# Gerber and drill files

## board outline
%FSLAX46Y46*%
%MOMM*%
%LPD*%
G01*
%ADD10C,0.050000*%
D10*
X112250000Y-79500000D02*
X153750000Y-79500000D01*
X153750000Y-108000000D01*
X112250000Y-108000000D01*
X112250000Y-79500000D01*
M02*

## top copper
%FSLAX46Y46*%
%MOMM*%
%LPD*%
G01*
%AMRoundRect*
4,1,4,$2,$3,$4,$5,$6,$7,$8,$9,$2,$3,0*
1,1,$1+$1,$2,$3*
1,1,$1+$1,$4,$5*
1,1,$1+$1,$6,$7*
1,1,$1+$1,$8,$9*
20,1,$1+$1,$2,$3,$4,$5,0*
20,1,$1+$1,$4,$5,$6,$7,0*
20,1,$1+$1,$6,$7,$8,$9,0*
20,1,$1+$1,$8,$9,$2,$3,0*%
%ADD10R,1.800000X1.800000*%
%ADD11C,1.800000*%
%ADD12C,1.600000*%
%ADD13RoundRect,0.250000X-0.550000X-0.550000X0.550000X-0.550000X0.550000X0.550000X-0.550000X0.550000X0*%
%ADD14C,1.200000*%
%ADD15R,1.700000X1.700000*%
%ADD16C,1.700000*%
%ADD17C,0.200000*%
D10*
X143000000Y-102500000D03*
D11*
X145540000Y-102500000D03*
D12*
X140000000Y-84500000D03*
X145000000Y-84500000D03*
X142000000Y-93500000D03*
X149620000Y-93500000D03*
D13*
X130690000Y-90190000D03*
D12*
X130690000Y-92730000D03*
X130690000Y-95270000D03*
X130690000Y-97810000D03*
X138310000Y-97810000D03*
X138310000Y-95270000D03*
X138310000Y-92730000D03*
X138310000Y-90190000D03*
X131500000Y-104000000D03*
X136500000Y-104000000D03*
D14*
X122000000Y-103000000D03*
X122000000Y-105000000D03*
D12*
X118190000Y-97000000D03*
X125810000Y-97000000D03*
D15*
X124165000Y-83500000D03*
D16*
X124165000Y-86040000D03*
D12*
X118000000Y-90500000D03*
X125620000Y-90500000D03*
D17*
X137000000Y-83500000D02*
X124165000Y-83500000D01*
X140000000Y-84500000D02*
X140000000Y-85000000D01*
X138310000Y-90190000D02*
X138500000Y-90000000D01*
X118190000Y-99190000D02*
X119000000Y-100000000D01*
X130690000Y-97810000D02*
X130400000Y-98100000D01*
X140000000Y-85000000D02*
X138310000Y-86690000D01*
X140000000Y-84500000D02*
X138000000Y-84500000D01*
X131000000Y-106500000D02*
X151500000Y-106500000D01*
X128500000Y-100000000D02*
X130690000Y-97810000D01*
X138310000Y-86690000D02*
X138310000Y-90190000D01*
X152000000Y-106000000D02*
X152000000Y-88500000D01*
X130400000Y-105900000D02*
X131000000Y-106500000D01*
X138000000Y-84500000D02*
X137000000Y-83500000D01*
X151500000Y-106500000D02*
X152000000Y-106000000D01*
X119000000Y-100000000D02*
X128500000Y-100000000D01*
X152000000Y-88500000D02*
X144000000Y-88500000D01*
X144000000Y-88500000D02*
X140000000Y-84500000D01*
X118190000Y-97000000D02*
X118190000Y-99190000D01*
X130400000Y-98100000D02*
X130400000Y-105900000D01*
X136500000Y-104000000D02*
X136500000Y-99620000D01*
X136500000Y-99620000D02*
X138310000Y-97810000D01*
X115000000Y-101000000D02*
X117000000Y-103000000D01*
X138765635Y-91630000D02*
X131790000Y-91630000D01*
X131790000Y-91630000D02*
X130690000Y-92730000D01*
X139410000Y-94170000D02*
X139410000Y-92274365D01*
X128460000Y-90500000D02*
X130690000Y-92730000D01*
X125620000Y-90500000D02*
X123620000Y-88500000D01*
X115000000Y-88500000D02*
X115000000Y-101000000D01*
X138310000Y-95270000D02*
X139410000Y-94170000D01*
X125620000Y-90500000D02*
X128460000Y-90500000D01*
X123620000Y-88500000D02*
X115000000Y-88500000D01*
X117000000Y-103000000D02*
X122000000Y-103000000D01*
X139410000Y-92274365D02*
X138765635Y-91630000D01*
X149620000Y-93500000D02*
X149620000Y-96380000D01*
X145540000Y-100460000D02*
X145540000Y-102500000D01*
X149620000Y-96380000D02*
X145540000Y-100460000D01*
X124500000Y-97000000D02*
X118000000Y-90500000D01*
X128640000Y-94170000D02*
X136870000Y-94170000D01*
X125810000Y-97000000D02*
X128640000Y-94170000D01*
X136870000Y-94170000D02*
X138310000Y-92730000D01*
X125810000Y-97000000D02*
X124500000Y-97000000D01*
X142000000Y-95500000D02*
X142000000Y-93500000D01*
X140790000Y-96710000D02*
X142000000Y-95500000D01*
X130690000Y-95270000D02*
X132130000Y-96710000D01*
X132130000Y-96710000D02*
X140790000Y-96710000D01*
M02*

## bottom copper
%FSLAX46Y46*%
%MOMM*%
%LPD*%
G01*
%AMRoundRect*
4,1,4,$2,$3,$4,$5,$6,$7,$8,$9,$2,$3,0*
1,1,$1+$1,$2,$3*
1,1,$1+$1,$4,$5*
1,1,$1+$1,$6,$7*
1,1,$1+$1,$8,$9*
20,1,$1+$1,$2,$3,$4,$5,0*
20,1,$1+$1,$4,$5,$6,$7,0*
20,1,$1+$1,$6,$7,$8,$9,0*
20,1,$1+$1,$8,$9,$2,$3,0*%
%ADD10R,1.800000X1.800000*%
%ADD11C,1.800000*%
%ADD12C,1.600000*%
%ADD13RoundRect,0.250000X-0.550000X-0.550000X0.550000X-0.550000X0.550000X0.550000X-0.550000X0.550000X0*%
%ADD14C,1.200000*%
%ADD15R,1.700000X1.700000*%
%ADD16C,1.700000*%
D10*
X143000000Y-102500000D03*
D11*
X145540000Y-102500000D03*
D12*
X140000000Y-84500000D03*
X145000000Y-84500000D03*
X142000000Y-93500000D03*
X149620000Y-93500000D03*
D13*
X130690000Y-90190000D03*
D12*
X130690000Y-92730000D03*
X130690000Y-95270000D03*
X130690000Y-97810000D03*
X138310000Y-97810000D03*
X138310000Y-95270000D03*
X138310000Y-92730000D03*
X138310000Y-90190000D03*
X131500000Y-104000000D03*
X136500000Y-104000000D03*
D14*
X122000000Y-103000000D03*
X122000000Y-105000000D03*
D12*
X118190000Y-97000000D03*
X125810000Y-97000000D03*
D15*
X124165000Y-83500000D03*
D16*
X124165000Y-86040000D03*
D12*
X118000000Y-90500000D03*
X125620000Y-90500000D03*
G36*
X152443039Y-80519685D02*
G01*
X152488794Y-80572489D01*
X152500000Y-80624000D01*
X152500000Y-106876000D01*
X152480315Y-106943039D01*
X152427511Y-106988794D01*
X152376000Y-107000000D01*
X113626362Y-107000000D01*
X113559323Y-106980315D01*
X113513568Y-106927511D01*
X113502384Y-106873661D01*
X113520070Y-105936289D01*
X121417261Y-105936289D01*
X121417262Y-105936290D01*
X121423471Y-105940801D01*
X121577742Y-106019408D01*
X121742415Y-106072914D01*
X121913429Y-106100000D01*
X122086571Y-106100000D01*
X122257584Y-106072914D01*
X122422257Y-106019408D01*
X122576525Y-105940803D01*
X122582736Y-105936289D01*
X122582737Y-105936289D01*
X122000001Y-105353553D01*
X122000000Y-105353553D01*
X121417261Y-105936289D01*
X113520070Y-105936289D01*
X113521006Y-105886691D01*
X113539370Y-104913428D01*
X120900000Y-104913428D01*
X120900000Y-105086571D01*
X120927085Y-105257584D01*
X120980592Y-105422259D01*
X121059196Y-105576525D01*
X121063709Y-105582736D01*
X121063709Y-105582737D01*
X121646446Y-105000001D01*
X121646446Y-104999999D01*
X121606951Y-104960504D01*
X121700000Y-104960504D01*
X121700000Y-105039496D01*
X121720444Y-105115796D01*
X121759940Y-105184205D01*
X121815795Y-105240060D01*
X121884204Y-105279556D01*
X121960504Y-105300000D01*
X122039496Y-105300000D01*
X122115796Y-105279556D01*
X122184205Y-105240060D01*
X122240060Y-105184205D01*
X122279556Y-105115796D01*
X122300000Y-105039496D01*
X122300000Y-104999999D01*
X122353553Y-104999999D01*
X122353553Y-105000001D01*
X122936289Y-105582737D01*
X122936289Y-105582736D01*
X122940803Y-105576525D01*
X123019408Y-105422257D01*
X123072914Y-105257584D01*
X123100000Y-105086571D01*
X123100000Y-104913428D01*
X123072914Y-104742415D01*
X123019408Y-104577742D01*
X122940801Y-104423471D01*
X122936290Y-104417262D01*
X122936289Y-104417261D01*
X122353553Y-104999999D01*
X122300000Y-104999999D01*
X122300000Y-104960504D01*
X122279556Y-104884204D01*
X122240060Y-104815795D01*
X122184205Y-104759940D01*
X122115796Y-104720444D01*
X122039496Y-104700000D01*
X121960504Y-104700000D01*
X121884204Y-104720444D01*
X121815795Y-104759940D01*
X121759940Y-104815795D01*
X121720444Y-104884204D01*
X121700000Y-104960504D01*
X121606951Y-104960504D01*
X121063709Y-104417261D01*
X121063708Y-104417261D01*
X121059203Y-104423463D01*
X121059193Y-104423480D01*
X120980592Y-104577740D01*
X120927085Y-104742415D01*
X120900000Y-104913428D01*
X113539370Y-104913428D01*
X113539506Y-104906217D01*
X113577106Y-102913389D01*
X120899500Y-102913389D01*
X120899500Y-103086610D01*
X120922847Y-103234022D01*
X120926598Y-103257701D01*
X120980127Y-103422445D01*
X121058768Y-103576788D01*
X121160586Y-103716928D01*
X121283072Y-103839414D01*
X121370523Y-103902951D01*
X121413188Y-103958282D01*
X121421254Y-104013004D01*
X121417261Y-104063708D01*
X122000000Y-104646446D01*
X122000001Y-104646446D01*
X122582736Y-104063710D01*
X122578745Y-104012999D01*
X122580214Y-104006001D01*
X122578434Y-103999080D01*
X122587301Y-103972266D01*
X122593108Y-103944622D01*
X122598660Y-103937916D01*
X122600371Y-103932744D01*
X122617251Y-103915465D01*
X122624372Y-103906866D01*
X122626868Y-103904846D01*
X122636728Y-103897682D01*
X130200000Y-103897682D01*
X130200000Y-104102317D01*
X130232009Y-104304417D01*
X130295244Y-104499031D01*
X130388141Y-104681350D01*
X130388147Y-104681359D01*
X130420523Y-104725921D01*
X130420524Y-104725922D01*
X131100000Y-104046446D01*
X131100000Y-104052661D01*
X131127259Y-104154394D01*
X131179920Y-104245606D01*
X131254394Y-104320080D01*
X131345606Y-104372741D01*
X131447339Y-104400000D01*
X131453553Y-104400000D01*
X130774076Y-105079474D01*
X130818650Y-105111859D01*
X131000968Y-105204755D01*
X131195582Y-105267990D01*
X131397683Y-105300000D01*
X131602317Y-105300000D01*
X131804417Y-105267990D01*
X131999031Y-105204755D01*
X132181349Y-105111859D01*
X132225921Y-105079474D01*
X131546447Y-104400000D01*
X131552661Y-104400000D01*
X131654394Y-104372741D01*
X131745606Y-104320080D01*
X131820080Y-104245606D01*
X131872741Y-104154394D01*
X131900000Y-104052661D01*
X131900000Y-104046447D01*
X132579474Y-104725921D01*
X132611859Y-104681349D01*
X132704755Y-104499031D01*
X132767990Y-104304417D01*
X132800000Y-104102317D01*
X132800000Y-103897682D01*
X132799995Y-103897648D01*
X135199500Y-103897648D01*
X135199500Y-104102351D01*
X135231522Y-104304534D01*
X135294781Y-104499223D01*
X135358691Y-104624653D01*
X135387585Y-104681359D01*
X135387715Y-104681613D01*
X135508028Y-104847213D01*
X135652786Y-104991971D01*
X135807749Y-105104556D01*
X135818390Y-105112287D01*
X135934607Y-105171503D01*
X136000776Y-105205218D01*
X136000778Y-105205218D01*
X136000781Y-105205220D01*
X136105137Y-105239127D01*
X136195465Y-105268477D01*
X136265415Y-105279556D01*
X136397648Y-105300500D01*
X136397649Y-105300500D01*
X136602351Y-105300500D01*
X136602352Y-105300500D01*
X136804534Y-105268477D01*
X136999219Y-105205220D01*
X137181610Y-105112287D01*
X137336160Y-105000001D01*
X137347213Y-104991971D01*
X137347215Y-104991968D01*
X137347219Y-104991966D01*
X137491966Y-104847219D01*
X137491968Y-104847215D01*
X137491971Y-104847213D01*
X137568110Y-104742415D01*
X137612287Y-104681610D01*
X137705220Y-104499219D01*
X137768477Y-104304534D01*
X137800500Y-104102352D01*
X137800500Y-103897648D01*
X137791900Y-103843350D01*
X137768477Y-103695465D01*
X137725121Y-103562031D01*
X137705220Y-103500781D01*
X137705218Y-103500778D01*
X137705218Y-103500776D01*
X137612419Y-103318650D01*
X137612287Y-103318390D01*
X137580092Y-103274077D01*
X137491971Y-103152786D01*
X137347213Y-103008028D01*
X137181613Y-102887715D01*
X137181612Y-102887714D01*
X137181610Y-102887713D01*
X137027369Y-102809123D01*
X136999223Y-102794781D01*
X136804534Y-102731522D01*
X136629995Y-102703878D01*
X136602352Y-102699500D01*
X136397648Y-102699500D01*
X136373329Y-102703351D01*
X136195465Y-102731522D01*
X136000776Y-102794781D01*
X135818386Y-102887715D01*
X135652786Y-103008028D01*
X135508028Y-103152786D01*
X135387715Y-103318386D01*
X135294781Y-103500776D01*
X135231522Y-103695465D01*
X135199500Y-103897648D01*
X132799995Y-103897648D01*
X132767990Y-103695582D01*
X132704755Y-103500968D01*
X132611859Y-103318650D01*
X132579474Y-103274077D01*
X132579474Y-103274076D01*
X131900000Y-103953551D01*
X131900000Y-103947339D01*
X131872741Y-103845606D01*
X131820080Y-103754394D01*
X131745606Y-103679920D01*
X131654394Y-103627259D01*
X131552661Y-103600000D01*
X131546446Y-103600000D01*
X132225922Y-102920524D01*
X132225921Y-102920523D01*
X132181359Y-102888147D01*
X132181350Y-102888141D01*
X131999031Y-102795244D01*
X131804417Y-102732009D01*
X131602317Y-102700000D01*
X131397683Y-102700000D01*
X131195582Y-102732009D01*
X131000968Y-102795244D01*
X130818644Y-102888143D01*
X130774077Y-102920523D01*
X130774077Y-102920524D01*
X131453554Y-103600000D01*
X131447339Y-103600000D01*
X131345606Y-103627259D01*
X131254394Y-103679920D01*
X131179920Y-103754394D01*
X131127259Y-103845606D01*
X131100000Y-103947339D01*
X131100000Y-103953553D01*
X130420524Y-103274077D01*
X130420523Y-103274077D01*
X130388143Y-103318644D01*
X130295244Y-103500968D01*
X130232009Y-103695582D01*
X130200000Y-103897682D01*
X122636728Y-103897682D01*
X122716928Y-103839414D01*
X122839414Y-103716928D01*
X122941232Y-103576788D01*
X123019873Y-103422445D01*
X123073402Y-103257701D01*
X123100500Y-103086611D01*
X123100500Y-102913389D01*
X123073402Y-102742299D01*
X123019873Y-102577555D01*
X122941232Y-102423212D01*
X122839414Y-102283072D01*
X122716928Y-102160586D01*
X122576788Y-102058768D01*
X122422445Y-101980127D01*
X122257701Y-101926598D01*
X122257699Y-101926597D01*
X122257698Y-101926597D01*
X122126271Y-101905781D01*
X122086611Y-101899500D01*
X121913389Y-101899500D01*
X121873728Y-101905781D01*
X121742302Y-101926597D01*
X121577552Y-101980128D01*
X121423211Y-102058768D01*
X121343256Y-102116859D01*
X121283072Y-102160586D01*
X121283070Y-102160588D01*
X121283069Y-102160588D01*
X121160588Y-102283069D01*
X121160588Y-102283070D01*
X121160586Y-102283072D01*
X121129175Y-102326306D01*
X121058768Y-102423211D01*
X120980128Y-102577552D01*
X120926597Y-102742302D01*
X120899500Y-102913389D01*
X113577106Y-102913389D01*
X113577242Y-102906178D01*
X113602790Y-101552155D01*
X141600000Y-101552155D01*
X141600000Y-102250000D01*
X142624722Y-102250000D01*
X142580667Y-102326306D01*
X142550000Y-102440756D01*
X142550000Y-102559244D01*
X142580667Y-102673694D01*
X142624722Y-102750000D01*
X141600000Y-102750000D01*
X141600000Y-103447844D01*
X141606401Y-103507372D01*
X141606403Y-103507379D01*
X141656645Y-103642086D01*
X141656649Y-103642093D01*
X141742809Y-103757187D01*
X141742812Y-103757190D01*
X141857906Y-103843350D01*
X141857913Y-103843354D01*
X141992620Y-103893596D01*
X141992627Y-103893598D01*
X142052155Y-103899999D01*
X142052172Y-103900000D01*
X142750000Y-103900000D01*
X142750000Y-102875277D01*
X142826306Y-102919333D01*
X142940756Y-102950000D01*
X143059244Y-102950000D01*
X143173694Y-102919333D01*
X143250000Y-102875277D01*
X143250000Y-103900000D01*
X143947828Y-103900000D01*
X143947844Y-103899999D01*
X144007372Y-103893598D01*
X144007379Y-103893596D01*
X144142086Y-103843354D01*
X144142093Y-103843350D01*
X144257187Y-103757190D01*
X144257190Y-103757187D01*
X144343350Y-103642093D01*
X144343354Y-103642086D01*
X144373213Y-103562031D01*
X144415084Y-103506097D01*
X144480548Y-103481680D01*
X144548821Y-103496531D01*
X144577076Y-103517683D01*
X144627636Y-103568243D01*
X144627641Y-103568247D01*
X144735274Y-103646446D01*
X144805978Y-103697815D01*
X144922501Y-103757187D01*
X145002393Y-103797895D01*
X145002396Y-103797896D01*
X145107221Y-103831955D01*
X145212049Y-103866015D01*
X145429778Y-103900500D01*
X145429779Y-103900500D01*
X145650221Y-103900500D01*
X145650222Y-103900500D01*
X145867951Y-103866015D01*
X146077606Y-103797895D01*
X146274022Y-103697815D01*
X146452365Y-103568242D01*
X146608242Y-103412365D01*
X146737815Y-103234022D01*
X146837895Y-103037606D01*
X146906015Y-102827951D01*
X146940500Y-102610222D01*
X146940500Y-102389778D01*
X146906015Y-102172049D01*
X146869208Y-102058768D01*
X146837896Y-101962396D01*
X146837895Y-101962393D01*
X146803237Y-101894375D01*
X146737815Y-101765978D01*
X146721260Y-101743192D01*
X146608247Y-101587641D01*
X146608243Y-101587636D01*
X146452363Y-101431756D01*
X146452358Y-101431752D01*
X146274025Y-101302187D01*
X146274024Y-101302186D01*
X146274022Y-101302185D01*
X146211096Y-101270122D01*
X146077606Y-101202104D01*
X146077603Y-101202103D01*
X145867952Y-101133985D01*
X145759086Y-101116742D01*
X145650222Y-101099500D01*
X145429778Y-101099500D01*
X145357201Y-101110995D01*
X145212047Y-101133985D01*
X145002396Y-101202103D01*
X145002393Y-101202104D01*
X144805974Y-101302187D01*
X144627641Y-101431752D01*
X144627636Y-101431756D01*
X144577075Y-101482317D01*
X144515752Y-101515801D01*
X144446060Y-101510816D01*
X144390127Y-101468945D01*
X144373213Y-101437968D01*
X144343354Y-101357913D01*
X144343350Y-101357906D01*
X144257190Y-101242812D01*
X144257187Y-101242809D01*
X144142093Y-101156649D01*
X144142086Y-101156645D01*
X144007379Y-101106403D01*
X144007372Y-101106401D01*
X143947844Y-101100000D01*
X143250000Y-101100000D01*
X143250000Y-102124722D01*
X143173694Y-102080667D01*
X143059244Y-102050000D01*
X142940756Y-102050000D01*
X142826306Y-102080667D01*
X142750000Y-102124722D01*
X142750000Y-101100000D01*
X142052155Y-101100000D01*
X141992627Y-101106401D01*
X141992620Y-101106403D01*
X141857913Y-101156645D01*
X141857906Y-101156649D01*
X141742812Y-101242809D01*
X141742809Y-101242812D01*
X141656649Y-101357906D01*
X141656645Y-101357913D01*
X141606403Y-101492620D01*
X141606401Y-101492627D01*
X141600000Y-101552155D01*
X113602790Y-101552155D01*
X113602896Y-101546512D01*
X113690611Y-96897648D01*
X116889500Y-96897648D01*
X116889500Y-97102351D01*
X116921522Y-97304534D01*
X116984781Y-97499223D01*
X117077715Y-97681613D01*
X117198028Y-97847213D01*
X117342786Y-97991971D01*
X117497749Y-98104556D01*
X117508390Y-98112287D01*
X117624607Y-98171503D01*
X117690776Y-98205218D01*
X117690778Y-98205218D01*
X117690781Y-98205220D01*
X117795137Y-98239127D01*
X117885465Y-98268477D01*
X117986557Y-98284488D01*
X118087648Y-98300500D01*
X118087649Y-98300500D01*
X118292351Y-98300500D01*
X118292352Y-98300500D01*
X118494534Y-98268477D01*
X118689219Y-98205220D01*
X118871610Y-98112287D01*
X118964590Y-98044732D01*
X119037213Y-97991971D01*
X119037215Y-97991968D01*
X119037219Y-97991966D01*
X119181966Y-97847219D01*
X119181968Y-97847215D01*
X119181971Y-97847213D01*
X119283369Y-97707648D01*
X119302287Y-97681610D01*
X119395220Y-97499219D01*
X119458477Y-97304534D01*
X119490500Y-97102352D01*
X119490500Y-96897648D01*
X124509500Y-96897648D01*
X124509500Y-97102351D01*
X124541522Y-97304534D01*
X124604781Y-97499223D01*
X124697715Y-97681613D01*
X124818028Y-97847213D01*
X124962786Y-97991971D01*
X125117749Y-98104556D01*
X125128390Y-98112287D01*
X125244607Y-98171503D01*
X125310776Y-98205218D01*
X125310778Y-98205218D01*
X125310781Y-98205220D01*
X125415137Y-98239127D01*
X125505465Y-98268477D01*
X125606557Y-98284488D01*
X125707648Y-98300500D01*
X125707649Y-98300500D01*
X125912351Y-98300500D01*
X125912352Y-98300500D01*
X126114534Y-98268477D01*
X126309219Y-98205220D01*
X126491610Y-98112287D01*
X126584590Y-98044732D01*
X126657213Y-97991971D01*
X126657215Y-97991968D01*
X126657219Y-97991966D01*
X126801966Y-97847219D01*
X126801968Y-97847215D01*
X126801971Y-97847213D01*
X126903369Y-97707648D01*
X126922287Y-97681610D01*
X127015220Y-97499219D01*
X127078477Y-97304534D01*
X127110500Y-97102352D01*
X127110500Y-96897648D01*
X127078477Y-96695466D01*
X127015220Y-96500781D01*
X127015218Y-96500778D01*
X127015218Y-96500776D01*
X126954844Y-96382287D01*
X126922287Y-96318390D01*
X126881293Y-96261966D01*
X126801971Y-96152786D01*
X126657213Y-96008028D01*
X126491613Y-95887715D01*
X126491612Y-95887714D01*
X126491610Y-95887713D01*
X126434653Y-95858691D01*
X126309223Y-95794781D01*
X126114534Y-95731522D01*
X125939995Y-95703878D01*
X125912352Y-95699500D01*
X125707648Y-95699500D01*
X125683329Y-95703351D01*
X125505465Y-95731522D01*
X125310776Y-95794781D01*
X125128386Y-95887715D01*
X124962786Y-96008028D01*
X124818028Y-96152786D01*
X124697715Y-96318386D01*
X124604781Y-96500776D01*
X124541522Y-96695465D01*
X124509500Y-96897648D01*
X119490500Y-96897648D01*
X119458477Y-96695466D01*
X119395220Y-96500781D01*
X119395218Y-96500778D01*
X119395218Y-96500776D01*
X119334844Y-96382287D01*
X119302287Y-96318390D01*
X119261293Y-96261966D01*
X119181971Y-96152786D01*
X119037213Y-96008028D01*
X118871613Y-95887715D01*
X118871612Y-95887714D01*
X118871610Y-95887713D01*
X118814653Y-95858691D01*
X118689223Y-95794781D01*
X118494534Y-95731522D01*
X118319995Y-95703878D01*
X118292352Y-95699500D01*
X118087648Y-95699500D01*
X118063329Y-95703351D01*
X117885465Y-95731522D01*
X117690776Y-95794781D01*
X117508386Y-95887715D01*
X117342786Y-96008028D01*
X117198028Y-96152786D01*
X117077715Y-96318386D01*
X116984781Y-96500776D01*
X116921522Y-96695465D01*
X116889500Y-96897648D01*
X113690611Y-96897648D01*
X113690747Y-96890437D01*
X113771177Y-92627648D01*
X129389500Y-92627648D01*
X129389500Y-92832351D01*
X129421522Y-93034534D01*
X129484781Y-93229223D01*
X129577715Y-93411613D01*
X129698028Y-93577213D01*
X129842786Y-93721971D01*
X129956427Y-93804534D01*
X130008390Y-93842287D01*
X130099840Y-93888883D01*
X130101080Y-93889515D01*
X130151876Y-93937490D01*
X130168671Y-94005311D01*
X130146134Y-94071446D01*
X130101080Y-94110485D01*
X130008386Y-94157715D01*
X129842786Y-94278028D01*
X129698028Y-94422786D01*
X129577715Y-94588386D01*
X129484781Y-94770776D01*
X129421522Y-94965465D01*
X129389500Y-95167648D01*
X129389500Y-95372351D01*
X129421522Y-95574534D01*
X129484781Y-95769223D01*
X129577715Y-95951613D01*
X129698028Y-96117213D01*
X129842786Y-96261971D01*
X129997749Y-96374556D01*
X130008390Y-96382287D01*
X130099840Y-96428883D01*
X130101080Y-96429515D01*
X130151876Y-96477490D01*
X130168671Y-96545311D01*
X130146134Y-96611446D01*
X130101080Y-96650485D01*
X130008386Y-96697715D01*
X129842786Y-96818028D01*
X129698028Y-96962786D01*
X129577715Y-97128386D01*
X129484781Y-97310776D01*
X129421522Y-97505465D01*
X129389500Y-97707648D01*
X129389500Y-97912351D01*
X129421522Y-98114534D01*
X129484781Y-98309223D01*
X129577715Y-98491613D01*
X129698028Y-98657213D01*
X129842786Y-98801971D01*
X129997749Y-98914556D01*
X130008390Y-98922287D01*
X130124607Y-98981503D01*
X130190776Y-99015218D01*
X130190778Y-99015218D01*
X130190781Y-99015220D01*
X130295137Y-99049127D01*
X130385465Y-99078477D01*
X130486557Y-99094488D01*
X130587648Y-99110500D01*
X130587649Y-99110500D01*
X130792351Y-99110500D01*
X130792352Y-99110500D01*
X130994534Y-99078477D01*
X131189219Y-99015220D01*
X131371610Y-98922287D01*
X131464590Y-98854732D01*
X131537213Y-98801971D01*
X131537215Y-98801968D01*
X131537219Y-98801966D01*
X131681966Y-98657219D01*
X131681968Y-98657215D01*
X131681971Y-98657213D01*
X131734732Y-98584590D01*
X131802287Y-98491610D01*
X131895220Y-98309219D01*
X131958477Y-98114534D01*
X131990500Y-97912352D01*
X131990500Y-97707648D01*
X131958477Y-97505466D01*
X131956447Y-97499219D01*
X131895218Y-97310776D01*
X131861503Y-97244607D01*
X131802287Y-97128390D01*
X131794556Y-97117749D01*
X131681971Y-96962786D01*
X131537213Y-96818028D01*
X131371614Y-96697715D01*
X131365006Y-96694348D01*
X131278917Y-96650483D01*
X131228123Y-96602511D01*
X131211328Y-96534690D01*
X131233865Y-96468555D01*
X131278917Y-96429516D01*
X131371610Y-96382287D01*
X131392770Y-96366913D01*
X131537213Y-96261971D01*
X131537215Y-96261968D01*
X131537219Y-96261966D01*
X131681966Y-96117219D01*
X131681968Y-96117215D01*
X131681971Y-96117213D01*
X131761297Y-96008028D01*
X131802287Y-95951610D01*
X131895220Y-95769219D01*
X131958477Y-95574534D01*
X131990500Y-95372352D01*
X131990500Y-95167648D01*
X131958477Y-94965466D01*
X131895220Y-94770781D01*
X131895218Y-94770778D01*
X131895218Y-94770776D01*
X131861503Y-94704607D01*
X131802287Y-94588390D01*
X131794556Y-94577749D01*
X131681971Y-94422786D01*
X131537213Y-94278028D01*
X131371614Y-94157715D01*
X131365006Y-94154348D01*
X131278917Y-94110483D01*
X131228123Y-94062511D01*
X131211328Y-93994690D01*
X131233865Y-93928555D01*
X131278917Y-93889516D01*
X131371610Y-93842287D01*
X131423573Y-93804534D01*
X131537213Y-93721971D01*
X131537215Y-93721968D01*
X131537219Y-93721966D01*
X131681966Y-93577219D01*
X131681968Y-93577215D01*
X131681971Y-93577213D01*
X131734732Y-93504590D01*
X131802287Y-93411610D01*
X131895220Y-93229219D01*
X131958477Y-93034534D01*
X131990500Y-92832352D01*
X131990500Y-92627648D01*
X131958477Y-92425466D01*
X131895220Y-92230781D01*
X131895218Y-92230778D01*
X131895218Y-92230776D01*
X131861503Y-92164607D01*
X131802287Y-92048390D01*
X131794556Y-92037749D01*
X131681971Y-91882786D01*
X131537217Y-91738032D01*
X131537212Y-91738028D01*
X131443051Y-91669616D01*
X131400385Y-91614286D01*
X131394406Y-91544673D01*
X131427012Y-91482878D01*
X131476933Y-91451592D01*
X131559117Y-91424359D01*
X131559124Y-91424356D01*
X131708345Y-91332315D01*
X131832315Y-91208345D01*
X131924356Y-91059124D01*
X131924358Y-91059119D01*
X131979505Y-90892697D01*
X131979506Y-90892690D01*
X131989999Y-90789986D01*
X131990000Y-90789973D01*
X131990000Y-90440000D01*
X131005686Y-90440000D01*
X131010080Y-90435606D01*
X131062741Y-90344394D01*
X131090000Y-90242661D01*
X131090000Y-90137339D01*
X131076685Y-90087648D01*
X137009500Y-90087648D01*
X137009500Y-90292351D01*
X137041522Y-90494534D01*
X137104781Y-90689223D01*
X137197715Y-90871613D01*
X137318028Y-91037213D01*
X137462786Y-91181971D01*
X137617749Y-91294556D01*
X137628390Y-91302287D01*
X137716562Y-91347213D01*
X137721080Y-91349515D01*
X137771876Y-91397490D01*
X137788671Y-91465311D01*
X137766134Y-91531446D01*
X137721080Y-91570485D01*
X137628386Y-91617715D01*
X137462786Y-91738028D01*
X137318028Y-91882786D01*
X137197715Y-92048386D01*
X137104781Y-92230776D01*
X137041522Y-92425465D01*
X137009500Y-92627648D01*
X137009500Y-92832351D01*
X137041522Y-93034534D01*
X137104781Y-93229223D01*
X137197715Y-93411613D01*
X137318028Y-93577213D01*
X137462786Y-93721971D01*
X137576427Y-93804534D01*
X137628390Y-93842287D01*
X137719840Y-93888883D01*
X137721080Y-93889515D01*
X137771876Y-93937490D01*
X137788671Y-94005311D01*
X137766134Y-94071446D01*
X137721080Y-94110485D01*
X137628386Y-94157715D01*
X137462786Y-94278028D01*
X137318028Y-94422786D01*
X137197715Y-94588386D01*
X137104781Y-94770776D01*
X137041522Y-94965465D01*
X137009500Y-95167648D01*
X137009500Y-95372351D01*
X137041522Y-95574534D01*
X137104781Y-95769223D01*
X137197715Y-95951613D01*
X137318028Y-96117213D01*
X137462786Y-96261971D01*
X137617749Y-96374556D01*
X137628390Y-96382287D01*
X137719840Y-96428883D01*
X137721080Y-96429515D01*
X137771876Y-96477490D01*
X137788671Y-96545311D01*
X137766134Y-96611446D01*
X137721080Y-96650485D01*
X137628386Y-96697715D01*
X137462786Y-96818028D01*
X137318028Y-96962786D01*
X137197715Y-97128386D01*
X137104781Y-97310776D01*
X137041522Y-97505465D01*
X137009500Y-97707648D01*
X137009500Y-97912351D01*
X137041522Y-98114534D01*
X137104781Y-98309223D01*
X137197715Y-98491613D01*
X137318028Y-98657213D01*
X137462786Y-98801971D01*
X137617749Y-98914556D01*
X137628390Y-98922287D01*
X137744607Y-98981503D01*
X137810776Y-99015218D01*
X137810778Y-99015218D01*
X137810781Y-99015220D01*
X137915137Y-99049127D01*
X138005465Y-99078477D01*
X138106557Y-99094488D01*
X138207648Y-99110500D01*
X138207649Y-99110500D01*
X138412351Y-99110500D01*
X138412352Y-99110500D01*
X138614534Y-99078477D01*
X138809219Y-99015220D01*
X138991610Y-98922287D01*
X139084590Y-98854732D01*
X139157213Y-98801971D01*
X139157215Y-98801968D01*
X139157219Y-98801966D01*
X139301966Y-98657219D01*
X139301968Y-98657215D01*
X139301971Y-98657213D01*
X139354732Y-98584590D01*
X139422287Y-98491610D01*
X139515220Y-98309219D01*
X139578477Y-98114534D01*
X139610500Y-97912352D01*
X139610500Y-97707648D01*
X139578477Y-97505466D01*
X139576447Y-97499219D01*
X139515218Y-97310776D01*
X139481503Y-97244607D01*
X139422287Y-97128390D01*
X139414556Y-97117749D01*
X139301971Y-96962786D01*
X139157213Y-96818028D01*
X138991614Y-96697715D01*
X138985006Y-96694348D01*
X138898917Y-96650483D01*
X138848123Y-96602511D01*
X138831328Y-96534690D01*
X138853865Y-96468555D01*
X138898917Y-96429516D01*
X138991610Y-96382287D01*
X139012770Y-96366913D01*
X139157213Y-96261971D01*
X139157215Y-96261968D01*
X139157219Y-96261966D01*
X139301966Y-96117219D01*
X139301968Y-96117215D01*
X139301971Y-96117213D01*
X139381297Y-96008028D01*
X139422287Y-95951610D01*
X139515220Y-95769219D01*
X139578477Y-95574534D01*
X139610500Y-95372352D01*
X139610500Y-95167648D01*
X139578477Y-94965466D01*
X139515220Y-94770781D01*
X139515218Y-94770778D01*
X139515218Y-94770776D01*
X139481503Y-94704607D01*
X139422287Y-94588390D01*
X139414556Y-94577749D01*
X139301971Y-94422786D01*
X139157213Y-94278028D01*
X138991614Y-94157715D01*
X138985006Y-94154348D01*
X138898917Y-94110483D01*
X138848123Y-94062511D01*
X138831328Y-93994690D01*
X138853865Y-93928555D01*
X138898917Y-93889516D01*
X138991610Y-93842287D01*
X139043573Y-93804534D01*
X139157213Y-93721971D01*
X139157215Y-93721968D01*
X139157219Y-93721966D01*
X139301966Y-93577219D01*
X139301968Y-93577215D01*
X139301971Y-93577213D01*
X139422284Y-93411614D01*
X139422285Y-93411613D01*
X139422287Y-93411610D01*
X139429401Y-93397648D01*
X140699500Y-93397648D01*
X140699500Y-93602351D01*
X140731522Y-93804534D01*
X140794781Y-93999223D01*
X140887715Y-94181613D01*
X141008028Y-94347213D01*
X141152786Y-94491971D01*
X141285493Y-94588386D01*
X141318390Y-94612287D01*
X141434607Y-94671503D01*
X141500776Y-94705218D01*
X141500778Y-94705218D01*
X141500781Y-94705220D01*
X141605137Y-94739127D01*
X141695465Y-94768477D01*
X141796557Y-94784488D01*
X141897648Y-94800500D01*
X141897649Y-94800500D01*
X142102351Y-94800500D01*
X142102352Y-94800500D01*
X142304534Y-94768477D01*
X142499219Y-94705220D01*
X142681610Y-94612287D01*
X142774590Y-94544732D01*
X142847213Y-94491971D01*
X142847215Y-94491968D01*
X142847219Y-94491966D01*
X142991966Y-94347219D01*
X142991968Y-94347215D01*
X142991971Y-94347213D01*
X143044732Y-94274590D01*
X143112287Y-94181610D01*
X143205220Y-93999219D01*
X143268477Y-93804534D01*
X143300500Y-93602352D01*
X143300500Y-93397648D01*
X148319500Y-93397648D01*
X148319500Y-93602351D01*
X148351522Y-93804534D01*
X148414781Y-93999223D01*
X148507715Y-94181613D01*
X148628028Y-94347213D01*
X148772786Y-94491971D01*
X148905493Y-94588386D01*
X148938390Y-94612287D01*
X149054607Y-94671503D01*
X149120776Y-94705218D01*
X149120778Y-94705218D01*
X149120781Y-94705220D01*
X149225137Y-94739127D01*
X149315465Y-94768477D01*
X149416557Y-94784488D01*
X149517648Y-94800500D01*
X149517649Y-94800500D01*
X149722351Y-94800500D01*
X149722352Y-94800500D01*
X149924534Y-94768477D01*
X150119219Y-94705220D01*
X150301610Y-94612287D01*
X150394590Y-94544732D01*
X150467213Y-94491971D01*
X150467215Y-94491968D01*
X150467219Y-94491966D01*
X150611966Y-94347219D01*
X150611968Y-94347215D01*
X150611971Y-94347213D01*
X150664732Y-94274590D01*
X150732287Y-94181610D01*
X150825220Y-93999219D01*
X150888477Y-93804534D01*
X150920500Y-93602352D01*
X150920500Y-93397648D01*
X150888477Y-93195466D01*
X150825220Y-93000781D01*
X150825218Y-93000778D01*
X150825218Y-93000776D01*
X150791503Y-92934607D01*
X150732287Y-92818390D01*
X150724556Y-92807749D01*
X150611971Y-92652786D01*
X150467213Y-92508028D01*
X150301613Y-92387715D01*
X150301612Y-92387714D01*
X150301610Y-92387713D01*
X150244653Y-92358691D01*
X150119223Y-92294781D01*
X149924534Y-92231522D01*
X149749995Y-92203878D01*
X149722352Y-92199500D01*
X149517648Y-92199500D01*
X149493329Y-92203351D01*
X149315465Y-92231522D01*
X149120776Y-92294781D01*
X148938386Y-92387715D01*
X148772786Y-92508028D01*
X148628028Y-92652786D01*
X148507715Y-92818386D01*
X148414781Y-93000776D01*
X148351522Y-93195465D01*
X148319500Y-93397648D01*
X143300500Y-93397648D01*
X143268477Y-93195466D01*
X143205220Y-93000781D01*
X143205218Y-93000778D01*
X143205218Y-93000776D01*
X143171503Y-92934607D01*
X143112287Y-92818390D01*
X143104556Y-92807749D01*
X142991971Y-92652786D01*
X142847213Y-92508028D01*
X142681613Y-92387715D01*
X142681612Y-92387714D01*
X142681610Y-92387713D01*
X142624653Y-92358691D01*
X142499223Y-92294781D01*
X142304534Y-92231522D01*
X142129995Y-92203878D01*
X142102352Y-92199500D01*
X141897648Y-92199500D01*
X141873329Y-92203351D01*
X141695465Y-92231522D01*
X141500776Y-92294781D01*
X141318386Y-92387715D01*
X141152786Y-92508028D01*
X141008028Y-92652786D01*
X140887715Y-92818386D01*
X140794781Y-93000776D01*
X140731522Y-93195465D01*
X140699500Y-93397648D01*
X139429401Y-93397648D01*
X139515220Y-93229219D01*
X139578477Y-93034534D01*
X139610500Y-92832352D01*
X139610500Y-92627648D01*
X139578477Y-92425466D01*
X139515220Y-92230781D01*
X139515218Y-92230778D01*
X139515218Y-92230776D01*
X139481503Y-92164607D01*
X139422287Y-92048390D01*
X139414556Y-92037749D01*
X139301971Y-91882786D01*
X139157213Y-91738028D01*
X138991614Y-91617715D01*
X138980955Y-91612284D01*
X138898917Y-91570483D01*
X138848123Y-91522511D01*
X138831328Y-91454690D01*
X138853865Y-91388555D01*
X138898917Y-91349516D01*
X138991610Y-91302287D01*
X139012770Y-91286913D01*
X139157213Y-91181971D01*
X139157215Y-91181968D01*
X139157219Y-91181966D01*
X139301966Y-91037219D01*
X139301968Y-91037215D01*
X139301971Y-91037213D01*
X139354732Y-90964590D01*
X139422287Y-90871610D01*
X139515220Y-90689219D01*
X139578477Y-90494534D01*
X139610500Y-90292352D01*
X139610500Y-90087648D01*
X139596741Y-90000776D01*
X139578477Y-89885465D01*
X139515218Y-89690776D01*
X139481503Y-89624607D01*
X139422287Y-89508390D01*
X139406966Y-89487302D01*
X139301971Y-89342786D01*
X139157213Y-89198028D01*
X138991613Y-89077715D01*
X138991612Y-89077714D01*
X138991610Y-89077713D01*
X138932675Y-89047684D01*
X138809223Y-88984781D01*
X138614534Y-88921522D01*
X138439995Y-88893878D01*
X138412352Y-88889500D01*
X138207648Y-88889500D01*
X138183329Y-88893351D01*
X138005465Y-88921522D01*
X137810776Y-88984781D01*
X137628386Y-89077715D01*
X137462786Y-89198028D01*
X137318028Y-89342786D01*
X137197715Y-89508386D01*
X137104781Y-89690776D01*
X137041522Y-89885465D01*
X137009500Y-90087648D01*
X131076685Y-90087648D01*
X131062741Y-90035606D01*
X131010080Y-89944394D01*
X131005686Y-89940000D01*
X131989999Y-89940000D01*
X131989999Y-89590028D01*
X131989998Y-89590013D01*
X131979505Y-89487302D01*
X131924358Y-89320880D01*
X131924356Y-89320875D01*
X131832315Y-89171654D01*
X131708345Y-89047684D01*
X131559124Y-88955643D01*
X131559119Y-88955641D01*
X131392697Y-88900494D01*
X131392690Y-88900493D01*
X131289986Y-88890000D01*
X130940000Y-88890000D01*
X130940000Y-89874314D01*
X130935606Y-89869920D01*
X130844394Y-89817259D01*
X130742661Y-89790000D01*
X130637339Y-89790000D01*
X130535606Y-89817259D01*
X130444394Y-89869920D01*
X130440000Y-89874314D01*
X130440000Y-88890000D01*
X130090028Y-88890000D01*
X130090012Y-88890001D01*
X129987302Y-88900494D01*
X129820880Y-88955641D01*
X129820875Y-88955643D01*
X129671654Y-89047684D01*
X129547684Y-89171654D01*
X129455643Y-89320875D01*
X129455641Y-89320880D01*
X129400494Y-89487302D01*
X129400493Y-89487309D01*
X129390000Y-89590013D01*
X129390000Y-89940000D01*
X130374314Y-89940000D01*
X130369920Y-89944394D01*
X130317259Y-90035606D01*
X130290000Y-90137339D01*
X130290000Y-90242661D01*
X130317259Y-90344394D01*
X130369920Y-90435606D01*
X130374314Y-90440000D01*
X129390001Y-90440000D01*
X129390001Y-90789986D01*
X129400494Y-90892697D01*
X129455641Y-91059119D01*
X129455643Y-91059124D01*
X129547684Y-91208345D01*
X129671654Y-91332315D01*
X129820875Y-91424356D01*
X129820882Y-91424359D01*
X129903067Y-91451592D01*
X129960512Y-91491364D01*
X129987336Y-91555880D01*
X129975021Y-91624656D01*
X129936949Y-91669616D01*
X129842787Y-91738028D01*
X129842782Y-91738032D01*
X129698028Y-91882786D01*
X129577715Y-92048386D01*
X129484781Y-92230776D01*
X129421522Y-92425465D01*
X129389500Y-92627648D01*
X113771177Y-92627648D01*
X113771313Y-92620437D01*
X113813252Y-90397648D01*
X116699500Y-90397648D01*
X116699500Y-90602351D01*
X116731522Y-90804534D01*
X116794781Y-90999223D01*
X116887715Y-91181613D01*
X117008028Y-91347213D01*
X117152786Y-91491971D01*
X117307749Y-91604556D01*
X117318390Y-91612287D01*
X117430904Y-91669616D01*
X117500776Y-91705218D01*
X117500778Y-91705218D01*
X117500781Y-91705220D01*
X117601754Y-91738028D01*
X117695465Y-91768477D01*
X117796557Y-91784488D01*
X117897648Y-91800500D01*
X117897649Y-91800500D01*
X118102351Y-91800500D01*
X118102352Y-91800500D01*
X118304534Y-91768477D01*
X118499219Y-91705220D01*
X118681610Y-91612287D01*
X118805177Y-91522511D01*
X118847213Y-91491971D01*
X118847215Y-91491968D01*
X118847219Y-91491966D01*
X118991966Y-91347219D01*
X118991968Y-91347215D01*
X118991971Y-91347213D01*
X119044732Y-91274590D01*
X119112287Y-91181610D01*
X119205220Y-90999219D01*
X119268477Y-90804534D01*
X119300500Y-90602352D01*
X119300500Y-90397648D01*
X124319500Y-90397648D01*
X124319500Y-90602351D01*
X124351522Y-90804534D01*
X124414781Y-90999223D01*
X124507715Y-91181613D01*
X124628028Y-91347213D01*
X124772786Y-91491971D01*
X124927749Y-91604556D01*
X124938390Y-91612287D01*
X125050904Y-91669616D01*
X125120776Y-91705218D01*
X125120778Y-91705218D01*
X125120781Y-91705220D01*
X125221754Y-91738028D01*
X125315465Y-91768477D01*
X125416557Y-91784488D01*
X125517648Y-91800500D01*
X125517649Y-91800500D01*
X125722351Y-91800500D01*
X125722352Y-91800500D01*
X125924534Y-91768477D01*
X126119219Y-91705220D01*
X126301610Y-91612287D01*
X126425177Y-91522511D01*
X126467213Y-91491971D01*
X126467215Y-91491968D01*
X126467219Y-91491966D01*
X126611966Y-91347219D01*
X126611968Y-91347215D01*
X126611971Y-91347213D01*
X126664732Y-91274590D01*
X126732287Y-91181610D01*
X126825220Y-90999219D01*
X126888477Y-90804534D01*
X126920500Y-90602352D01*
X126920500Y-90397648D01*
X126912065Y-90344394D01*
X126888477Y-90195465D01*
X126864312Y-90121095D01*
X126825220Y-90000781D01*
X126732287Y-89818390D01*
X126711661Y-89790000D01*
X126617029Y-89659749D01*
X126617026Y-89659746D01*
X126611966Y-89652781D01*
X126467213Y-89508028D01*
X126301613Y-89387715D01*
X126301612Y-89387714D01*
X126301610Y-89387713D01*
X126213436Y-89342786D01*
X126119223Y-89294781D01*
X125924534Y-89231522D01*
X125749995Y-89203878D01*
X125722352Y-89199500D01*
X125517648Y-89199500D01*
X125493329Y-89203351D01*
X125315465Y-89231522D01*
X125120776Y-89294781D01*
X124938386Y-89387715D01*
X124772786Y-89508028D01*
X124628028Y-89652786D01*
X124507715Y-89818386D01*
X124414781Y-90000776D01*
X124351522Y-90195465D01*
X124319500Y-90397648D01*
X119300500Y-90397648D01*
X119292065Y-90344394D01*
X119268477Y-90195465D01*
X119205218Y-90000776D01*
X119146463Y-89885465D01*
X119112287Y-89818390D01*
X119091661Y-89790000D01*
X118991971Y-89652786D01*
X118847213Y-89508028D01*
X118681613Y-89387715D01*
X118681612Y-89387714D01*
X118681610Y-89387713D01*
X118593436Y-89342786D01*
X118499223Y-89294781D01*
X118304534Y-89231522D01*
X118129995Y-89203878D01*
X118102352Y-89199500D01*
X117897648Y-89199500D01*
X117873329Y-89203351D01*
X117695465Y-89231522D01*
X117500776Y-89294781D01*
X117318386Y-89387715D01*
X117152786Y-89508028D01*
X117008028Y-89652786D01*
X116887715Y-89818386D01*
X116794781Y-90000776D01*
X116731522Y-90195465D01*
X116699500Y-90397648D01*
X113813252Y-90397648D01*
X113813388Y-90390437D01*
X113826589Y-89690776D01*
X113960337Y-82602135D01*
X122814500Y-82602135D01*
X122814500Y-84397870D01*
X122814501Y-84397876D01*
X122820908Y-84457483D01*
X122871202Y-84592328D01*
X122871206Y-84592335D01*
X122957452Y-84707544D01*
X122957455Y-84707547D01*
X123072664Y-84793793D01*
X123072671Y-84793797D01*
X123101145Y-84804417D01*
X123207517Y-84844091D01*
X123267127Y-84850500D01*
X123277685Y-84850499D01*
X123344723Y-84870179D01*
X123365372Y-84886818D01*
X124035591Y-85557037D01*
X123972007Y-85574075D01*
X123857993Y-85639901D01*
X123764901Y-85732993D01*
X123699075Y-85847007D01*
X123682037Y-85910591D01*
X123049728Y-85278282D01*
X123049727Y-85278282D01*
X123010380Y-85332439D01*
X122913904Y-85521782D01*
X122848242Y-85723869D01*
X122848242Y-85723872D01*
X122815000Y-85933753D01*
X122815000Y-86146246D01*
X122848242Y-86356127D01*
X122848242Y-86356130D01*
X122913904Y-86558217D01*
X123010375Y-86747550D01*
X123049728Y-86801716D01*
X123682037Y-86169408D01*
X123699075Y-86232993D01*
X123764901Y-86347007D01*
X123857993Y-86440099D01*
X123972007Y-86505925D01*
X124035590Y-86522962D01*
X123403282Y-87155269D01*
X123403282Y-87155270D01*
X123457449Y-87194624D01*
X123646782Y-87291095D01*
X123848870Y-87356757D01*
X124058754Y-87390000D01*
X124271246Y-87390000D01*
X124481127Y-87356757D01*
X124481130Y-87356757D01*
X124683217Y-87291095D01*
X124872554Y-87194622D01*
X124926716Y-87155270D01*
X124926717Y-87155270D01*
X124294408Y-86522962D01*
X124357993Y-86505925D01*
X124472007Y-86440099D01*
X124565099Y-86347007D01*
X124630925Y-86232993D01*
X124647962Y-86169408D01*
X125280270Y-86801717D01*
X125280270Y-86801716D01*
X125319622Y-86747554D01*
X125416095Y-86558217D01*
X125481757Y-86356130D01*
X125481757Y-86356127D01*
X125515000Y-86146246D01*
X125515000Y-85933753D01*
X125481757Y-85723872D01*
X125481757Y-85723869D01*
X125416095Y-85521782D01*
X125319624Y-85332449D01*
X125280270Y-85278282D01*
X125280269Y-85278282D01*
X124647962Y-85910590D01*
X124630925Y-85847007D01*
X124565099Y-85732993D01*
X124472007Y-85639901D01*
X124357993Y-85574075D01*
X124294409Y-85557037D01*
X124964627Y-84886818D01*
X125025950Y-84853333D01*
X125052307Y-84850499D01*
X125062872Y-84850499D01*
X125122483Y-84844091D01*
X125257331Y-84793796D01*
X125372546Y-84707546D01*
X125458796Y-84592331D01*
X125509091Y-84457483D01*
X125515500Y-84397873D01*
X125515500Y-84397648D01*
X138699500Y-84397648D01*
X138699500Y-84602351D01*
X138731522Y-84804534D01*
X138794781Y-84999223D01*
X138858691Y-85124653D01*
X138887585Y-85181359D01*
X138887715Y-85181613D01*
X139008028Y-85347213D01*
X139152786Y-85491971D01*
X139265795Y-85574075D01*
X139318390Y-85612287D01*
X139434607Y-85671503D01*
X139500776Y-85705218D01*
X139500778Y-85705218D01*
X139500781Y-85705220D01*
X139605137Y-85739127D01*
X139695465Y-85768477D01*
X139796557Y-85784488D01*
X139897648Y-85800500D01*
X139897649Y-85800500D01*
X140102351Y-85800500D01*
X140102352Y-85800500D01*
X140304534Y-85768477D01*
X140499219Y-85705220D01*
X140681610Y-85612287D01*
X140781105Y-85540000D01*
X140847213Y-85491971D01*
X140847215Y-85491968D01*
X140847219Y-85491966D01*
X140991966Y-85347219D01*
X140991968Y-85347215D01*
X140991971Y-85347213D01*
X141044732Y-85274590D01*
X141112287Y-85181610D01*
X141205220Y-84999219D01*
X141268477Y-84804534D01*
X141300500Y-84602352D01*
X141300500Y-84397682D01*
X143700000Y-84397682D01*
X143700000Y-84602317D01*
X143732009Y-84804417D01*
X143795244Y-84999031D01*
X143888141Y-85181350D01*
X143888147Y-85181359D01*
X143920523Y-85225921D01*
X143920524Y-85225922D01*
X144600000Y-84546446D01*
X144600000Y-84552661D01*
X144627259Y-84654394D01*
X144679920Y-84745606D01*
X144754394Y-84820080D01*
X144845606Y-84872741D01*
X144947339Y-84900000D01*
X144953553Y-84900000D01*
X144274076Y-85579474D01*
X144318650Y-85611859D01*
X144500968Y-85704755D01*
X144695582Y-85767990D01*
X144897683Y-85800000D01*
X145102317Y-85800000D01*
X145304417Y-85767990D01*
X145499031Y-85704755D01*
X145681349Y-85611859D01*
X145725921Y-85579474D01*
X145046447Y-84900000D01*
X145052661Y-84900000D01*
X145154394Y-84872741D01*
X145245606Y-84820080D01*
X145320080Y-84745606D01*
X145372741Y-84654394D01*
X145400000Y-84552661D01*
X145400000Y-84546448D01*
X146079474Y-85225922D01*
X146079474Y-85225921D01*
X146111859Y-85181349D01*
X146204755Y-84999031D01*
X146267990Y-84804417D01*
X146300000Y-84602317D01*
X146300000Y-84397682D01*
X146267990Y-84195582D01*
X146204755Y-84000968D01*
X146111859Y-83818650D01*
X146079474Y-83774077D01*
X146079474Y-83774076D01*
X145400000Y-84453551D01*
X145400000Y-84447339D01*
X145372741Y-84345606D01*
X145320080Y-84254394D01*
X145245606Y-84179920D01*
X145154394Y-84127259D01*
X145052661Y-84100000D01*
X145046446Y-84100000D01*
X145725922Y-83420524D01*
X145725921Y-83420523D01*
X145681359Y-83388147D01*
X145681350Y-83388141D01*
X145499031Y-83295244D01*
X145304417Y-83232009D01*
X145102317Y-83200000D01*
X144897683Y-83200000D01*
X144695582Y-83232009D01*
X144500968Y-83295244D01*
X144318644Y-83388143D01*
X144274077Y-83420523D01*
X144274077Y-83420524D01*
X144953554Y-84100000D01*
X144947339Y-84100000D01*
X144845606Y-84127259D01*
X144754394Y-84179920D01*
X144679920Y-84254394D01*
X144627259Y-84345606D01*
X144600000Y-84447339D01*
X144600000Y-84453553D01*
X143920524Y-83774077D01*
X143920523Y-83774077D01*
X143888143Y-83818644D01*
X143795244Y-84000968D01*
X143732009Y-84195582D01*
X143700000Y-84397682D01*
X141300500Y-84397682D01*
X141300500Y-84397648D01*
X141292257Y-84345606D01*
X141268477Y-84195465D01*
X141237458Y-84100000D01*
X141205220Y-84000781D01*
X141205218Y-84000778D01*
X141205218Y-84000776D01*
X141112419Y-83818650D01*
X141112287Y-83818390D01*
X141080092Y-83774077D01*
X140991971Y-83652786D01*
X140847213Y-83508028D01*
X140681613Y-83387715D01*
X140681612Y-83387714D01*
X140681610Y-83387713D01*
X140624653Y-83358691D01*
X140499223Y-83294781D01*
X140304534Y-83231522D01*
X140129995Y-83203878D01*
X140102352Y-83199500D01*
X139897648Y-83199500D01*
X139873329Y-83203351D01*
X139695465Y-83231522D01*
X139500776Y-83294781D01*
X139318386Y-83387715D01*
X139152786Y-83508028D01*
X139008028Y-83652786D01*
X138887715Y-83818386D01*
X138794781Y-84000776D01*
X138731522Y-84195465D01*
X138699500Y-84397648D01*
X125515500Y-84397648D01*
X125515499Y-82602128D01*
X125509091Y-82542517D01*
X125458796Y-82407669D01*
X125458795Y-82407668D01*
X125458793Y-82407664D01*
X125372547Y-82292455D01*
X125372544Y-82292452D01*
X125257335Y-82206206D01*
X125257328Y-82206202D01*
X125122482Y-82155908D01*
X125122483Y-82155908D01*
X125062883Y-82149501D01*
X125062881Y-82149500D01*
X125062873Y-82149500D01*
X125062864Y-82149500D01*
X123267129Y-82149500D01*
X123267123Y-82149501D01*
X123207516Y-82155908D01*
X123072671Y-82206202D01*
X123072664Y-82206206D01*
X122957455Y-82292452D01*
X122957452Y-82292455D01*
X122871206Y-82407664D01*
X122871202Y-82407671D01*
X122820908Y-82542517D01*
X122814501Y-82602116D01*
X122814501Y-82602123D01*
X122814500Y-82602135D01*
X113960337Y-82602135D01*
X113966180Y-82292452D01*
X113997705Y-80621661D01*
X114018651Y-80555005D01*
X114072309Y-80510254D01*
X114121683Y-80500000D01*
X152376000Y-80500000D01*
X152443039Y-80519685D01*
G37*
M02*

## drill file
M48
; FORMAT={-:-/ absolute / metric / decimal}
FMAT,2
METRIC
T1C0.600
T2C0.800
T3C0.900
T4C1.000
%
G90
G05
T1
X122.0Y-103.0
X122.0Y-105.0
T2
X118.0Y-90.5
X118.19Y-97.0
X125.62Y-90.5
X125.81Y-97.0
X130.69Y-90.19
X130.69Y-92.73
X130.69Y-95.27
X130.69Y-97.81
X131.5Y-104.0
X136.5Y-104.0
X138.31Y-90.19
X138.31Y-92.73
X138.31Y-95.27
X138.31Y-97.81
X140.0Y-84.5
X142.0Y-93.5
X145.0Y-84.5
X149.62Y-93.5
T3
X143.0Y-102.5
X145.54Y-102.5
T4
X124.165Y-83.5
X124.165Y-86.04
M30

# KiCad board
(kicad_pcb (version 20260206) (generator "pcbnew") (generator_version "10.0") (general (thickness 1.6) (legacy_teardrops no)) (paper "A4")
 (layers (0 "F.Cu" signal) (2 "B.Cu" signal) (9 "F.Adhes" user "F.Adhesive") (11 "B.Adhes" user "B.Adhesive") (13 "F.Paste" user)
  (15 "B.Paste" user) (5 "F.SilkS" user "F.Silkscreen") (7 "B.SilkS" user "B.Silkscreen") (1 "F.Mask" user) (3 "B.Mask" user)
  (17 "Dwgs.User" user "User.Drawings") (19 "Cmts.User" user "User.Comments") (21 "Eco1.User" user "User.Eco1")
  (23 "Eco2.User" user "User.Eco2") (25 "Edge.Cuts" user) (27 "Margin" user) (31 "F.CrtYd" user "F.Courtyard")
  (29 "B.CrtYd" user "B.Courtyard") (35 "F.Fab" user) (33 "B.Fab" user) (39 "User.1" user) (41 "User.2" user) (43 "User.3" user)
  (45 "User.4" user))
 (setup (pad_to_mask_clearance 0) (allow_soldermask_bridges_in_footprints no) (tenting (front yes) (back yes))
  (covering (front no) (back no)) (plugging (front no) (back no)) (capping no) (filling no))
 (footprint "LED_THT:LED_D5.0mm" (layer "F.Cu") (at 143 102.5)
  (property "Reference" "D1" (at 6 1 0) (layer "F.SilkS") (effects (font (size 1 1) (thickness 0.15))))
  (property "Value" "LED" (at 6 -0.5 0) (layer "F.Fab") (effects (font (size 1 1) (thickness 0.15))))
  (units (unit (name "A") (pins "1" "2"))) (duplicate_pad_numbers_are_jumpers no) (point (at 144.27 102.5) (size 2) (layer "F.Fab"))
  (pad "1" thru_hole rect (at 0 0) (size 1.8 1.8) (drill 0.9) (layers "*.Cu" "*.Mask") (remove_unused_layers no) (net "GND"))
  (pad "2" thru_hole circle (at 2.54 0) (size 1.8 1.8) (drill 0.9) (layers "*.Cu" "*.Mask") (remove_unused_layers no) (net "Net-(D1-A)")))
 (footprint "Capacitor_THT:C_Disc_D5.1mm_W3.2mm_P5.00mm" (layer "F.Cu") (at 140 84.5)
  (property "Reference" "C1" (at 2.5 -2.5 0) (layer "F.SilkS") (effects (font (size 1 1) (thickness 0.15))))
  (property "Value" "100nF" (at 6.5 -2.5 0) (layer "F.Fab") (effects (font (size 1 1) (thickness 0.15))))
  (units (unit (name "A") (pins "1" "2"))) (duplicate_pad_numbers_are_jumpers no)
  (pad "1" thru_hole circle (at 0 0) (size 1.6 1.6) (drill 0.8) (layers "*.Cu" "*.Mask") (remove_unused_layers no) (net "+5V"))
  (pad "2" thru_hole circle (at 5 0) (size 1.6 1.6) (drill 0.8) (layers "*.Cu" "*.Mask") (remove_unused_layers no) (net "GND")))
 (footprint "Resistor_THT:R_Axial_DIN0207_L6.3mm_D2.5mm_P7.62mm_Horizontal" (layer "F.Cu") (at 142 93.5)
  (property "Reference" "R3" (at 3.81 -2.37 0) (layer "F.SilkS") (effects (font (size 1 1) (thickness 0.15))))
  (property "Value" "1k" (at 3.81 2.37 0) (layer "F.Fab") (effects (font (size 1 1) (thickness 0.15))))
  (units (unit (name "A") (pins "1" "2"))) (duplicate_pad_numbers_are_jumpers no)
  (pad "1" thru_hole circle (at 0 0) (size 1.6 1.6) (drill 0.8) (layers "*.Cu" "*.Mask") (remove_unused_layers no) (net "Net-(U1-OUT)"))
  (pad "2" thru_hole circle (at 7.62 0) (size 1.6 1.6) (drill 0.8) (layers "*.Cu" "*.Mask") (remove_unused_layers no) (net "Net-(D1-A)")))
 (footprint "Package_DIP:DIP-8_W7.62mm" (layer "F.Cu") (at 130.69 90.19)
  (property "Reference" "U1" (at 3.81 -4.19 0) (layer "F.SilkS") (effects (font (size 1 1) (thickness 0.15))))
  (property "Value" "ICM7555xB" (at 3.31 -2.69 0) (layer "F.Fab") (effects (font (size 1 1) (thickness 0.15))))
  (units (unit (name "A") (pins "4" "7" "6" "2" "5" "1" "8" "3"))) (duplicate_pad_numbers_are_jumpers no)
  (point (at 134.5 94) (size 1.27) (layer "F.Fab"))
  (pad "1" thru_hole roundrect (at 0 0) (size 1.6 1.6) (drill 0.8) (layers "*.Cu" "*.Mask") (remove_unused_layers no)
   (roundrect_rratio 0.15625) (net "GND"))
  (pad "2" thru_hole circle (at 0 2.54) (size 1.6 1.6) (drill 0.8) (layers "*.Cu" "*.Mask") (remove_unused_layers no) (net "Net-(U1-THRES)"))
  (pad "3" thru_hole circle (at 0 5.08) (size 1.6 1.6) (drill 0.8) (layers "*.Cu" "*.Mask") (remove_unused_layers no) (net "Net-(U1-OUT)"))
  (pad "4" thru_hole circle (at 0 7.62) (size 1.6 1.6) (drill 0.8) (layers "*.Cu" "*.Mask") (remove_unused_layers no) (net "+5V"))
  (pad "5" thru_hole circle (at 7.62 7.62) (size 1.6 1.6) (drill 0.8) (layers "*.Cu" "*.Mask") (remove_unused_layers no)
   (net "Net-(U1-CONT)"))
  (pad "6" thru_hole circle (at 7.62 5.08) (size 1.6 1.6) (drill 0.8) (layers "*.Cu" "*.Mask") (remove_unused_layers no)
   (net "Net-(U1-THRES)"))
  (pad "7" thru_hole circle (at 7.62 2.54) (size 1.6 1.6) (drill 0.8) (layers "*.Cu" "*.Mask") (remove_unused_layers no)
   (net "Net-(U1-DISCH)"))
  (pad "8" thru_hole circle (at 7.62 0) (size 1.6 1.6) (drill 0.8) (layers "*.Cu" "*.Mask") (remove_unused_layers no) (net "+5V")))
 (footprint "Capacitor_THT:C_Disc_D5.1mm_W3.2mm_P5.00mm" (layer "F.Cu") (at 131.5 104)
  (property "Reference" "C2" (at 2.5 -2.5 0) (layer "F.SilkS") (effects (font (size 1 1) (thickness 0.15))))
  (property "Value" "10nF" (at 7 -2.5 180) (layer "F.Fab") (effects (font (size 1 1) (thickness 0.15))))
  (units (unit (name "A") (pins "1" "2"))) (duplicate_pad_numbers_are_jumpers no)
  (pad "1" thru_hole circle (at 0 0) (size 1.6 1.6) (drill 0.8) (layers "*.Cu" "*.Mask") (remove_unused_layers no) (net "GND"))
  (pad "2" thru_hole circle (at 5 0) (size 1.6 1.6) (drill 0.8) (layers "*.Cu" "*.Mask") (remove_unused_layers no) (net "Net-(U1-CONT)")))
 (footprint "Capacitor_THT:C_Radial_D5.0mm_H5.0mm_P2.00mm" (layer "F.Cu") (at 122 103 -90)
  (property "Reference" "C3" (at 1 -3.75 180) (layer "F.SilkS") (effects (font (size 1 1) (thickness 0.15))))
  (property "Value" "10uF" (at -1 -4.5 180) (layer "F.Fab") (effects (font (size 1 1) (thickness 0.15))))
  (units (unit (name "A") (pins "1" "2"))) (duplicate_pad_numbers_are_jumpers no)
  (pad "1" thru_hole circle (at 0 0 270) (size 1.2 1.2) (drill 0.6) (layers "*.Cu" "*.Mask") (remove_unused_layers no)
   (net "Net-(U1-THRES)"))
  (pad "2" thru_hole circle (at 2 0 270) (size 1.2 1.2) (drill 0.6) (layers "*.Cu" "*.Mask") (remove_unused_layers no) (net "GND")))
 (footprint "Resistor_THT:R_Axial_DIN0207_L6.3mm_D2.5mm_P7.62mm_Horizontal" (layer "F.Cu") (at 118.19 97)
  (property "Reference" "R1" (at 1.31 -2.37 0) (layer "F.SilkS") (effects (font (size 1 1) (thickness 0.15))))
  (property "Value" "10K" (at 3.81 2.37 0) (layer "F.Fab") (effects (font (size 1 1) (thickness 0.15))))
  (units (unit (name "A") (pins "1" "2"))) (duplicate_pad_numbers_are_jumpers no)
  (pad "1" thru_hole circle (at 0 0) (size 1.6 1.6) (drill 0.8) (layers "*.Cu" "*.Mask") (remove_unused_layers no) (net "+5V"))
  (pad "2" thru_hole circle (at 7.62 0) (size 1.6 1.6) (drill 0.8) (layers "*.Cu" "*.Mask") (remove_unused_layers no) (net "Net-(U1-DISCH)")))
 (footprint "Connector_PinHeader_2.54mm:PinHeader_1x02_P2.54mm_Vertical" (layer "F.Cu") (at 124.165 83.5)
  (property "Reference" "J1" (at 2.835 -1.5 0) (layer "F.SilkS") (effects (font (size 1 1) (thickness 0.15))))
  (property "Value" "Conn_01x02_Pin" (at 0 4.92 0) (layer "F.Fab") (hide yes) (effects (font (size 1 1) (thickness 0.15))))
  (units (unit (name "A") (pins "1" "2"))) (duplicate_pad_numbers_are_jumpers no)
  (pad "1" thru_hole rect (at 0 0) (size 1.7 1.7) (drill 1) (layers "*.Cu" "*.Mask") (remove_unused_layers no) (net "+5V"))
  (pad "2" thru_hole circle (at 0 2.54) (size 1.7 1.7) (drill 1) (layers "*.Cu" "*.Mask") (remove_unused_layers no) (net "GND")))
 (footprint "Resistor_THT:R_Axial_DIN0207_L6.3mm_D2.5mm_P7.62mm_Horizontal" (layer "F.Cu") (at 118 90.5)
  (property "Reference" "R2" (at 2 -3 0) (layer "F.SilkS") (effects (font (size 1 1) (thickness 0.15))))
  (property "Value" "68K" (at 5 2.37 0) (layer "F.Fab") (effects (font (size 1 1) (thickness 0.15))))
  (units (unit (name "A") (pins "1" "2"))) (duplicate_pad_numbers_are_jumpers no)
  (pad "1" thru_hole circle (at 0 0) (size 1.6 1.6) (drill 0.8) (layers "*.Cu" "*.Mask") (remove_unused_layers no) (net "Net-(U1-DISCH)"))
  (pad "2" thru_hole circle (at 7.62 0) (size 1.6 1.6) (drill 0.8) (layers "*.Cu" "*.Mask") (remove_unused_layers no) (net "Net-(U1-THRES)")))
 (gr_rect (start 112.25 79.5) (end 153.75 108) (stroke (width 0.05) (type default)) (fill no) (layer "Edge.Cuts"))
 (segment (start 137 83.5) (end 124.165 83.5) (width 0.2) (layer "F.Cu") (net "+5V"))
 (segment (start 140 84.5) (end 140 85) (width 0.2) (layer "F.Cu") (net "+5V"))
 (segment (start 138.31 90.19) (end 138.5 90) (width 0.2) (layer "F.Cu") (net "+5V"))
 (segment (start 118.19 99.19) (end 119 100) (width 0.2) (layer "F.Cu") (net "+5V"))
 (segment (start 130.69 97.81) (end 130.4 98.1) (width 0.2) (layer "F.Cu") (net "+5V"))
 (segment (start 140 85) (end 138.31 86.69) (width 0.2) (layer "F.Cu") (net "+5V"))
 (segment (start 140 84.5) (end 138 84.5) (width 0.2) (layer "F.Cu") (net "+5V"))
 (segment (start 131 106.5) (end 151.5 106.5) (width 0.2) (layer "F.Cu") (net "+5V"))
 (segment (start 128.5 100) (end 130.69 97.81) (width 0.2) (layer "F.Cu") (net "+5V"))
 (segment (start 138.31 86.69) (end 138.31 90.19) (width 0.2) (layer "F.Cu") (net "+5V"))
 (segment (start 152 106) (end 152 88.5) (width 0.2) (layer "F.Cu") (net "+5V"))
 (segment (start 130.4 105.9) (end 131 106.5) (width 0.2) (layer "F.Cu") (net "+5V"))
 (segment (start 138 84.5) (end 137 83.5) (width 0.2) (layer "F.Cu") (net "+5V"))
 (segment (start 151.5 106.5) (end 152 106) (width 0.2) (layer "F.Cu") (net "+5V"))
 (segment (start 119 100) (end 128.5 100) (width 0.2) (layer "F.Cu") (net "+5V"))
 (segment (start 152 88.5) (end 144 88.5) (width 0.2) (layer "F.Cu") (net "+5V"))
 (segment (start 144 88.5) (end 140 84.5) (width 0.2) (layer "F.Cu") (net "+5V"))
 (segment (start 118.19 97) (end 118.19 99.19) (width 0.2) (layer "F.Cu") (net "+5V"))
 (segment (start 130.4 98.1) (end 130.4 105.9) (width 0.2) (layer "F.Cu") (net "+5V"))
 (segment (start 136.5 104) (end 136.5 99.62) (width 0.2) (layer "F.Cu") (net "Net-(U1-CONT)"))
 (segment (start 136.5 99.62) (end 138.31 97.81) (width 0.2) (layer "F.Cu") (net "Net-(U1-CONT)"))
 (segment (start 115 101) (end 117 103) (width 0.2) (layer "F.Cu") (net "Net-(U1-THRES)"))
 (segment (start 138.765635 91.63) (end 131.79 91.63) (width 0.2) (layer "F.Cu") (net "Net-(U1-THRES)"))
 (segment (start 131.79 91.63) (end 130.69 92.73) (width 0.2) (layer "F.Cu") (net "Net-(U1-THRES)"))
 (segment (start 139.41 94.17) (end 139.41 92.274365) (width 0.2) (layer "F.Cu") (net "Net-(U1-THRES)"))
 (segment (start 128.46 90.5) (end 130.69 92.73) (width 0.2) (layer "F.Cu") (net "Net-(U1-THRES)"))
 (segment (start 125.62 90.5) (end 123.62 88.5) (width 0.2) (layer "F.Cu") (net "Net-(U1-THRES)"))
 (segment (start 115 88.5) (end 115 101) (width 0.2) (layer "F.Cu") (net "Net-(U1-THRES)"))
 (segment (start 138.31 95.27) (end 139.41 94.17) (width 0.2) (layer "F.Cu") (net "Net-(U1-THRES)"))
 (segment (start 125.62 90.5) (end 128.46 90.5) (width 0.2) (layer "F.Cu") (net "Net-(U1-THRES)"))
 (segment (start 123.62 88.5) (end 115 88.5) (width 0.2) (layer "F.Cu") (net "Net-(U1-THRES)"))
 (segment (start 117 103) (end 122 103) (width 0.2) (layer "F.Cu") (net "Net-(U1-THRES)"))
 (segment (start 139.41 92.274365) (end 138.765635 91.63) (width 0.2) (layer "F.Cu") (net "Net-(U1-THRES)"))
 (segment (start 149.62 93.5) (end 149.62 96.38) (width 0.2) (layer "F.Cu") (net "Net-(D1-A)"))
 (segment (start 145.54 100.46) (end 145.54 102.5) (width 0.2) (layer "F.Cu") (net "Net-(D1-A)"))
 (segment (start 149.62 96.38) (end 145.54 100.46) (width 0.2) (layer "F.Cu") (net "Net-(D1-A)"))
 (segment (start 124.5 97) (end 118 90.5) (width 0.2) (layer "F.Cu") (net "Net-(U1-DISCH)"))
 (segment (start 128.64 94.17) (end 136.87 94.17) (width 0.2) (layer "F.Cu") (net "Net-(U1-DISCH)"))
 (segment (start 125.81 97) (end 128.64 94.17) (width 0.2) (layer "F.Cu") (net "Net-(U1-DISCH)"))
 (segment (start 136.87 94.17) (end 138.31 92.73) (width 0.2) (layer "F.Cu") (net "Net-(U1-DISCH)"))
 (segment (start 125.81 97) (end 124.5 97) (width 0.2) (layer "F.Cu") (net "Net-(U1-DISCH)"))
 (segment (start 142 95.5) (end 142 93.5) (width 0.2) (layer "F.Cu") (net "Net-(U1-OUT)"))
 (segment (start 140.79 96.71) (end 142 95.5) (width 0.2) (layer "F.Cu") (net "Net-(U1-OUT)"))
 (segment (start 130.69 95.27) (end 132.13 96.71) (width 0.2) (layer "F.Cu") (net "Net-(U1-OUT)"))
 (segment (start 132.13 96.71) (end 140.79 96.71) (width 0.2) (layer "F.Cu") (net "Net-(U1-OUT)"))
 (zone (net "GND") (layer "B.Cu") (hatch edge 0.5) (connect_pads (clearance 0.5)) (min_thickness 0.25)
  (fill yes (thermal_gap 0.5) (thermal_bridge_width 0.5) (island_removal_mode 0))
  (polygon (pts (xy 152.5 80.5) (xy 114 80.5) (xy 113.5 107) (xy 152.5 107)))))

